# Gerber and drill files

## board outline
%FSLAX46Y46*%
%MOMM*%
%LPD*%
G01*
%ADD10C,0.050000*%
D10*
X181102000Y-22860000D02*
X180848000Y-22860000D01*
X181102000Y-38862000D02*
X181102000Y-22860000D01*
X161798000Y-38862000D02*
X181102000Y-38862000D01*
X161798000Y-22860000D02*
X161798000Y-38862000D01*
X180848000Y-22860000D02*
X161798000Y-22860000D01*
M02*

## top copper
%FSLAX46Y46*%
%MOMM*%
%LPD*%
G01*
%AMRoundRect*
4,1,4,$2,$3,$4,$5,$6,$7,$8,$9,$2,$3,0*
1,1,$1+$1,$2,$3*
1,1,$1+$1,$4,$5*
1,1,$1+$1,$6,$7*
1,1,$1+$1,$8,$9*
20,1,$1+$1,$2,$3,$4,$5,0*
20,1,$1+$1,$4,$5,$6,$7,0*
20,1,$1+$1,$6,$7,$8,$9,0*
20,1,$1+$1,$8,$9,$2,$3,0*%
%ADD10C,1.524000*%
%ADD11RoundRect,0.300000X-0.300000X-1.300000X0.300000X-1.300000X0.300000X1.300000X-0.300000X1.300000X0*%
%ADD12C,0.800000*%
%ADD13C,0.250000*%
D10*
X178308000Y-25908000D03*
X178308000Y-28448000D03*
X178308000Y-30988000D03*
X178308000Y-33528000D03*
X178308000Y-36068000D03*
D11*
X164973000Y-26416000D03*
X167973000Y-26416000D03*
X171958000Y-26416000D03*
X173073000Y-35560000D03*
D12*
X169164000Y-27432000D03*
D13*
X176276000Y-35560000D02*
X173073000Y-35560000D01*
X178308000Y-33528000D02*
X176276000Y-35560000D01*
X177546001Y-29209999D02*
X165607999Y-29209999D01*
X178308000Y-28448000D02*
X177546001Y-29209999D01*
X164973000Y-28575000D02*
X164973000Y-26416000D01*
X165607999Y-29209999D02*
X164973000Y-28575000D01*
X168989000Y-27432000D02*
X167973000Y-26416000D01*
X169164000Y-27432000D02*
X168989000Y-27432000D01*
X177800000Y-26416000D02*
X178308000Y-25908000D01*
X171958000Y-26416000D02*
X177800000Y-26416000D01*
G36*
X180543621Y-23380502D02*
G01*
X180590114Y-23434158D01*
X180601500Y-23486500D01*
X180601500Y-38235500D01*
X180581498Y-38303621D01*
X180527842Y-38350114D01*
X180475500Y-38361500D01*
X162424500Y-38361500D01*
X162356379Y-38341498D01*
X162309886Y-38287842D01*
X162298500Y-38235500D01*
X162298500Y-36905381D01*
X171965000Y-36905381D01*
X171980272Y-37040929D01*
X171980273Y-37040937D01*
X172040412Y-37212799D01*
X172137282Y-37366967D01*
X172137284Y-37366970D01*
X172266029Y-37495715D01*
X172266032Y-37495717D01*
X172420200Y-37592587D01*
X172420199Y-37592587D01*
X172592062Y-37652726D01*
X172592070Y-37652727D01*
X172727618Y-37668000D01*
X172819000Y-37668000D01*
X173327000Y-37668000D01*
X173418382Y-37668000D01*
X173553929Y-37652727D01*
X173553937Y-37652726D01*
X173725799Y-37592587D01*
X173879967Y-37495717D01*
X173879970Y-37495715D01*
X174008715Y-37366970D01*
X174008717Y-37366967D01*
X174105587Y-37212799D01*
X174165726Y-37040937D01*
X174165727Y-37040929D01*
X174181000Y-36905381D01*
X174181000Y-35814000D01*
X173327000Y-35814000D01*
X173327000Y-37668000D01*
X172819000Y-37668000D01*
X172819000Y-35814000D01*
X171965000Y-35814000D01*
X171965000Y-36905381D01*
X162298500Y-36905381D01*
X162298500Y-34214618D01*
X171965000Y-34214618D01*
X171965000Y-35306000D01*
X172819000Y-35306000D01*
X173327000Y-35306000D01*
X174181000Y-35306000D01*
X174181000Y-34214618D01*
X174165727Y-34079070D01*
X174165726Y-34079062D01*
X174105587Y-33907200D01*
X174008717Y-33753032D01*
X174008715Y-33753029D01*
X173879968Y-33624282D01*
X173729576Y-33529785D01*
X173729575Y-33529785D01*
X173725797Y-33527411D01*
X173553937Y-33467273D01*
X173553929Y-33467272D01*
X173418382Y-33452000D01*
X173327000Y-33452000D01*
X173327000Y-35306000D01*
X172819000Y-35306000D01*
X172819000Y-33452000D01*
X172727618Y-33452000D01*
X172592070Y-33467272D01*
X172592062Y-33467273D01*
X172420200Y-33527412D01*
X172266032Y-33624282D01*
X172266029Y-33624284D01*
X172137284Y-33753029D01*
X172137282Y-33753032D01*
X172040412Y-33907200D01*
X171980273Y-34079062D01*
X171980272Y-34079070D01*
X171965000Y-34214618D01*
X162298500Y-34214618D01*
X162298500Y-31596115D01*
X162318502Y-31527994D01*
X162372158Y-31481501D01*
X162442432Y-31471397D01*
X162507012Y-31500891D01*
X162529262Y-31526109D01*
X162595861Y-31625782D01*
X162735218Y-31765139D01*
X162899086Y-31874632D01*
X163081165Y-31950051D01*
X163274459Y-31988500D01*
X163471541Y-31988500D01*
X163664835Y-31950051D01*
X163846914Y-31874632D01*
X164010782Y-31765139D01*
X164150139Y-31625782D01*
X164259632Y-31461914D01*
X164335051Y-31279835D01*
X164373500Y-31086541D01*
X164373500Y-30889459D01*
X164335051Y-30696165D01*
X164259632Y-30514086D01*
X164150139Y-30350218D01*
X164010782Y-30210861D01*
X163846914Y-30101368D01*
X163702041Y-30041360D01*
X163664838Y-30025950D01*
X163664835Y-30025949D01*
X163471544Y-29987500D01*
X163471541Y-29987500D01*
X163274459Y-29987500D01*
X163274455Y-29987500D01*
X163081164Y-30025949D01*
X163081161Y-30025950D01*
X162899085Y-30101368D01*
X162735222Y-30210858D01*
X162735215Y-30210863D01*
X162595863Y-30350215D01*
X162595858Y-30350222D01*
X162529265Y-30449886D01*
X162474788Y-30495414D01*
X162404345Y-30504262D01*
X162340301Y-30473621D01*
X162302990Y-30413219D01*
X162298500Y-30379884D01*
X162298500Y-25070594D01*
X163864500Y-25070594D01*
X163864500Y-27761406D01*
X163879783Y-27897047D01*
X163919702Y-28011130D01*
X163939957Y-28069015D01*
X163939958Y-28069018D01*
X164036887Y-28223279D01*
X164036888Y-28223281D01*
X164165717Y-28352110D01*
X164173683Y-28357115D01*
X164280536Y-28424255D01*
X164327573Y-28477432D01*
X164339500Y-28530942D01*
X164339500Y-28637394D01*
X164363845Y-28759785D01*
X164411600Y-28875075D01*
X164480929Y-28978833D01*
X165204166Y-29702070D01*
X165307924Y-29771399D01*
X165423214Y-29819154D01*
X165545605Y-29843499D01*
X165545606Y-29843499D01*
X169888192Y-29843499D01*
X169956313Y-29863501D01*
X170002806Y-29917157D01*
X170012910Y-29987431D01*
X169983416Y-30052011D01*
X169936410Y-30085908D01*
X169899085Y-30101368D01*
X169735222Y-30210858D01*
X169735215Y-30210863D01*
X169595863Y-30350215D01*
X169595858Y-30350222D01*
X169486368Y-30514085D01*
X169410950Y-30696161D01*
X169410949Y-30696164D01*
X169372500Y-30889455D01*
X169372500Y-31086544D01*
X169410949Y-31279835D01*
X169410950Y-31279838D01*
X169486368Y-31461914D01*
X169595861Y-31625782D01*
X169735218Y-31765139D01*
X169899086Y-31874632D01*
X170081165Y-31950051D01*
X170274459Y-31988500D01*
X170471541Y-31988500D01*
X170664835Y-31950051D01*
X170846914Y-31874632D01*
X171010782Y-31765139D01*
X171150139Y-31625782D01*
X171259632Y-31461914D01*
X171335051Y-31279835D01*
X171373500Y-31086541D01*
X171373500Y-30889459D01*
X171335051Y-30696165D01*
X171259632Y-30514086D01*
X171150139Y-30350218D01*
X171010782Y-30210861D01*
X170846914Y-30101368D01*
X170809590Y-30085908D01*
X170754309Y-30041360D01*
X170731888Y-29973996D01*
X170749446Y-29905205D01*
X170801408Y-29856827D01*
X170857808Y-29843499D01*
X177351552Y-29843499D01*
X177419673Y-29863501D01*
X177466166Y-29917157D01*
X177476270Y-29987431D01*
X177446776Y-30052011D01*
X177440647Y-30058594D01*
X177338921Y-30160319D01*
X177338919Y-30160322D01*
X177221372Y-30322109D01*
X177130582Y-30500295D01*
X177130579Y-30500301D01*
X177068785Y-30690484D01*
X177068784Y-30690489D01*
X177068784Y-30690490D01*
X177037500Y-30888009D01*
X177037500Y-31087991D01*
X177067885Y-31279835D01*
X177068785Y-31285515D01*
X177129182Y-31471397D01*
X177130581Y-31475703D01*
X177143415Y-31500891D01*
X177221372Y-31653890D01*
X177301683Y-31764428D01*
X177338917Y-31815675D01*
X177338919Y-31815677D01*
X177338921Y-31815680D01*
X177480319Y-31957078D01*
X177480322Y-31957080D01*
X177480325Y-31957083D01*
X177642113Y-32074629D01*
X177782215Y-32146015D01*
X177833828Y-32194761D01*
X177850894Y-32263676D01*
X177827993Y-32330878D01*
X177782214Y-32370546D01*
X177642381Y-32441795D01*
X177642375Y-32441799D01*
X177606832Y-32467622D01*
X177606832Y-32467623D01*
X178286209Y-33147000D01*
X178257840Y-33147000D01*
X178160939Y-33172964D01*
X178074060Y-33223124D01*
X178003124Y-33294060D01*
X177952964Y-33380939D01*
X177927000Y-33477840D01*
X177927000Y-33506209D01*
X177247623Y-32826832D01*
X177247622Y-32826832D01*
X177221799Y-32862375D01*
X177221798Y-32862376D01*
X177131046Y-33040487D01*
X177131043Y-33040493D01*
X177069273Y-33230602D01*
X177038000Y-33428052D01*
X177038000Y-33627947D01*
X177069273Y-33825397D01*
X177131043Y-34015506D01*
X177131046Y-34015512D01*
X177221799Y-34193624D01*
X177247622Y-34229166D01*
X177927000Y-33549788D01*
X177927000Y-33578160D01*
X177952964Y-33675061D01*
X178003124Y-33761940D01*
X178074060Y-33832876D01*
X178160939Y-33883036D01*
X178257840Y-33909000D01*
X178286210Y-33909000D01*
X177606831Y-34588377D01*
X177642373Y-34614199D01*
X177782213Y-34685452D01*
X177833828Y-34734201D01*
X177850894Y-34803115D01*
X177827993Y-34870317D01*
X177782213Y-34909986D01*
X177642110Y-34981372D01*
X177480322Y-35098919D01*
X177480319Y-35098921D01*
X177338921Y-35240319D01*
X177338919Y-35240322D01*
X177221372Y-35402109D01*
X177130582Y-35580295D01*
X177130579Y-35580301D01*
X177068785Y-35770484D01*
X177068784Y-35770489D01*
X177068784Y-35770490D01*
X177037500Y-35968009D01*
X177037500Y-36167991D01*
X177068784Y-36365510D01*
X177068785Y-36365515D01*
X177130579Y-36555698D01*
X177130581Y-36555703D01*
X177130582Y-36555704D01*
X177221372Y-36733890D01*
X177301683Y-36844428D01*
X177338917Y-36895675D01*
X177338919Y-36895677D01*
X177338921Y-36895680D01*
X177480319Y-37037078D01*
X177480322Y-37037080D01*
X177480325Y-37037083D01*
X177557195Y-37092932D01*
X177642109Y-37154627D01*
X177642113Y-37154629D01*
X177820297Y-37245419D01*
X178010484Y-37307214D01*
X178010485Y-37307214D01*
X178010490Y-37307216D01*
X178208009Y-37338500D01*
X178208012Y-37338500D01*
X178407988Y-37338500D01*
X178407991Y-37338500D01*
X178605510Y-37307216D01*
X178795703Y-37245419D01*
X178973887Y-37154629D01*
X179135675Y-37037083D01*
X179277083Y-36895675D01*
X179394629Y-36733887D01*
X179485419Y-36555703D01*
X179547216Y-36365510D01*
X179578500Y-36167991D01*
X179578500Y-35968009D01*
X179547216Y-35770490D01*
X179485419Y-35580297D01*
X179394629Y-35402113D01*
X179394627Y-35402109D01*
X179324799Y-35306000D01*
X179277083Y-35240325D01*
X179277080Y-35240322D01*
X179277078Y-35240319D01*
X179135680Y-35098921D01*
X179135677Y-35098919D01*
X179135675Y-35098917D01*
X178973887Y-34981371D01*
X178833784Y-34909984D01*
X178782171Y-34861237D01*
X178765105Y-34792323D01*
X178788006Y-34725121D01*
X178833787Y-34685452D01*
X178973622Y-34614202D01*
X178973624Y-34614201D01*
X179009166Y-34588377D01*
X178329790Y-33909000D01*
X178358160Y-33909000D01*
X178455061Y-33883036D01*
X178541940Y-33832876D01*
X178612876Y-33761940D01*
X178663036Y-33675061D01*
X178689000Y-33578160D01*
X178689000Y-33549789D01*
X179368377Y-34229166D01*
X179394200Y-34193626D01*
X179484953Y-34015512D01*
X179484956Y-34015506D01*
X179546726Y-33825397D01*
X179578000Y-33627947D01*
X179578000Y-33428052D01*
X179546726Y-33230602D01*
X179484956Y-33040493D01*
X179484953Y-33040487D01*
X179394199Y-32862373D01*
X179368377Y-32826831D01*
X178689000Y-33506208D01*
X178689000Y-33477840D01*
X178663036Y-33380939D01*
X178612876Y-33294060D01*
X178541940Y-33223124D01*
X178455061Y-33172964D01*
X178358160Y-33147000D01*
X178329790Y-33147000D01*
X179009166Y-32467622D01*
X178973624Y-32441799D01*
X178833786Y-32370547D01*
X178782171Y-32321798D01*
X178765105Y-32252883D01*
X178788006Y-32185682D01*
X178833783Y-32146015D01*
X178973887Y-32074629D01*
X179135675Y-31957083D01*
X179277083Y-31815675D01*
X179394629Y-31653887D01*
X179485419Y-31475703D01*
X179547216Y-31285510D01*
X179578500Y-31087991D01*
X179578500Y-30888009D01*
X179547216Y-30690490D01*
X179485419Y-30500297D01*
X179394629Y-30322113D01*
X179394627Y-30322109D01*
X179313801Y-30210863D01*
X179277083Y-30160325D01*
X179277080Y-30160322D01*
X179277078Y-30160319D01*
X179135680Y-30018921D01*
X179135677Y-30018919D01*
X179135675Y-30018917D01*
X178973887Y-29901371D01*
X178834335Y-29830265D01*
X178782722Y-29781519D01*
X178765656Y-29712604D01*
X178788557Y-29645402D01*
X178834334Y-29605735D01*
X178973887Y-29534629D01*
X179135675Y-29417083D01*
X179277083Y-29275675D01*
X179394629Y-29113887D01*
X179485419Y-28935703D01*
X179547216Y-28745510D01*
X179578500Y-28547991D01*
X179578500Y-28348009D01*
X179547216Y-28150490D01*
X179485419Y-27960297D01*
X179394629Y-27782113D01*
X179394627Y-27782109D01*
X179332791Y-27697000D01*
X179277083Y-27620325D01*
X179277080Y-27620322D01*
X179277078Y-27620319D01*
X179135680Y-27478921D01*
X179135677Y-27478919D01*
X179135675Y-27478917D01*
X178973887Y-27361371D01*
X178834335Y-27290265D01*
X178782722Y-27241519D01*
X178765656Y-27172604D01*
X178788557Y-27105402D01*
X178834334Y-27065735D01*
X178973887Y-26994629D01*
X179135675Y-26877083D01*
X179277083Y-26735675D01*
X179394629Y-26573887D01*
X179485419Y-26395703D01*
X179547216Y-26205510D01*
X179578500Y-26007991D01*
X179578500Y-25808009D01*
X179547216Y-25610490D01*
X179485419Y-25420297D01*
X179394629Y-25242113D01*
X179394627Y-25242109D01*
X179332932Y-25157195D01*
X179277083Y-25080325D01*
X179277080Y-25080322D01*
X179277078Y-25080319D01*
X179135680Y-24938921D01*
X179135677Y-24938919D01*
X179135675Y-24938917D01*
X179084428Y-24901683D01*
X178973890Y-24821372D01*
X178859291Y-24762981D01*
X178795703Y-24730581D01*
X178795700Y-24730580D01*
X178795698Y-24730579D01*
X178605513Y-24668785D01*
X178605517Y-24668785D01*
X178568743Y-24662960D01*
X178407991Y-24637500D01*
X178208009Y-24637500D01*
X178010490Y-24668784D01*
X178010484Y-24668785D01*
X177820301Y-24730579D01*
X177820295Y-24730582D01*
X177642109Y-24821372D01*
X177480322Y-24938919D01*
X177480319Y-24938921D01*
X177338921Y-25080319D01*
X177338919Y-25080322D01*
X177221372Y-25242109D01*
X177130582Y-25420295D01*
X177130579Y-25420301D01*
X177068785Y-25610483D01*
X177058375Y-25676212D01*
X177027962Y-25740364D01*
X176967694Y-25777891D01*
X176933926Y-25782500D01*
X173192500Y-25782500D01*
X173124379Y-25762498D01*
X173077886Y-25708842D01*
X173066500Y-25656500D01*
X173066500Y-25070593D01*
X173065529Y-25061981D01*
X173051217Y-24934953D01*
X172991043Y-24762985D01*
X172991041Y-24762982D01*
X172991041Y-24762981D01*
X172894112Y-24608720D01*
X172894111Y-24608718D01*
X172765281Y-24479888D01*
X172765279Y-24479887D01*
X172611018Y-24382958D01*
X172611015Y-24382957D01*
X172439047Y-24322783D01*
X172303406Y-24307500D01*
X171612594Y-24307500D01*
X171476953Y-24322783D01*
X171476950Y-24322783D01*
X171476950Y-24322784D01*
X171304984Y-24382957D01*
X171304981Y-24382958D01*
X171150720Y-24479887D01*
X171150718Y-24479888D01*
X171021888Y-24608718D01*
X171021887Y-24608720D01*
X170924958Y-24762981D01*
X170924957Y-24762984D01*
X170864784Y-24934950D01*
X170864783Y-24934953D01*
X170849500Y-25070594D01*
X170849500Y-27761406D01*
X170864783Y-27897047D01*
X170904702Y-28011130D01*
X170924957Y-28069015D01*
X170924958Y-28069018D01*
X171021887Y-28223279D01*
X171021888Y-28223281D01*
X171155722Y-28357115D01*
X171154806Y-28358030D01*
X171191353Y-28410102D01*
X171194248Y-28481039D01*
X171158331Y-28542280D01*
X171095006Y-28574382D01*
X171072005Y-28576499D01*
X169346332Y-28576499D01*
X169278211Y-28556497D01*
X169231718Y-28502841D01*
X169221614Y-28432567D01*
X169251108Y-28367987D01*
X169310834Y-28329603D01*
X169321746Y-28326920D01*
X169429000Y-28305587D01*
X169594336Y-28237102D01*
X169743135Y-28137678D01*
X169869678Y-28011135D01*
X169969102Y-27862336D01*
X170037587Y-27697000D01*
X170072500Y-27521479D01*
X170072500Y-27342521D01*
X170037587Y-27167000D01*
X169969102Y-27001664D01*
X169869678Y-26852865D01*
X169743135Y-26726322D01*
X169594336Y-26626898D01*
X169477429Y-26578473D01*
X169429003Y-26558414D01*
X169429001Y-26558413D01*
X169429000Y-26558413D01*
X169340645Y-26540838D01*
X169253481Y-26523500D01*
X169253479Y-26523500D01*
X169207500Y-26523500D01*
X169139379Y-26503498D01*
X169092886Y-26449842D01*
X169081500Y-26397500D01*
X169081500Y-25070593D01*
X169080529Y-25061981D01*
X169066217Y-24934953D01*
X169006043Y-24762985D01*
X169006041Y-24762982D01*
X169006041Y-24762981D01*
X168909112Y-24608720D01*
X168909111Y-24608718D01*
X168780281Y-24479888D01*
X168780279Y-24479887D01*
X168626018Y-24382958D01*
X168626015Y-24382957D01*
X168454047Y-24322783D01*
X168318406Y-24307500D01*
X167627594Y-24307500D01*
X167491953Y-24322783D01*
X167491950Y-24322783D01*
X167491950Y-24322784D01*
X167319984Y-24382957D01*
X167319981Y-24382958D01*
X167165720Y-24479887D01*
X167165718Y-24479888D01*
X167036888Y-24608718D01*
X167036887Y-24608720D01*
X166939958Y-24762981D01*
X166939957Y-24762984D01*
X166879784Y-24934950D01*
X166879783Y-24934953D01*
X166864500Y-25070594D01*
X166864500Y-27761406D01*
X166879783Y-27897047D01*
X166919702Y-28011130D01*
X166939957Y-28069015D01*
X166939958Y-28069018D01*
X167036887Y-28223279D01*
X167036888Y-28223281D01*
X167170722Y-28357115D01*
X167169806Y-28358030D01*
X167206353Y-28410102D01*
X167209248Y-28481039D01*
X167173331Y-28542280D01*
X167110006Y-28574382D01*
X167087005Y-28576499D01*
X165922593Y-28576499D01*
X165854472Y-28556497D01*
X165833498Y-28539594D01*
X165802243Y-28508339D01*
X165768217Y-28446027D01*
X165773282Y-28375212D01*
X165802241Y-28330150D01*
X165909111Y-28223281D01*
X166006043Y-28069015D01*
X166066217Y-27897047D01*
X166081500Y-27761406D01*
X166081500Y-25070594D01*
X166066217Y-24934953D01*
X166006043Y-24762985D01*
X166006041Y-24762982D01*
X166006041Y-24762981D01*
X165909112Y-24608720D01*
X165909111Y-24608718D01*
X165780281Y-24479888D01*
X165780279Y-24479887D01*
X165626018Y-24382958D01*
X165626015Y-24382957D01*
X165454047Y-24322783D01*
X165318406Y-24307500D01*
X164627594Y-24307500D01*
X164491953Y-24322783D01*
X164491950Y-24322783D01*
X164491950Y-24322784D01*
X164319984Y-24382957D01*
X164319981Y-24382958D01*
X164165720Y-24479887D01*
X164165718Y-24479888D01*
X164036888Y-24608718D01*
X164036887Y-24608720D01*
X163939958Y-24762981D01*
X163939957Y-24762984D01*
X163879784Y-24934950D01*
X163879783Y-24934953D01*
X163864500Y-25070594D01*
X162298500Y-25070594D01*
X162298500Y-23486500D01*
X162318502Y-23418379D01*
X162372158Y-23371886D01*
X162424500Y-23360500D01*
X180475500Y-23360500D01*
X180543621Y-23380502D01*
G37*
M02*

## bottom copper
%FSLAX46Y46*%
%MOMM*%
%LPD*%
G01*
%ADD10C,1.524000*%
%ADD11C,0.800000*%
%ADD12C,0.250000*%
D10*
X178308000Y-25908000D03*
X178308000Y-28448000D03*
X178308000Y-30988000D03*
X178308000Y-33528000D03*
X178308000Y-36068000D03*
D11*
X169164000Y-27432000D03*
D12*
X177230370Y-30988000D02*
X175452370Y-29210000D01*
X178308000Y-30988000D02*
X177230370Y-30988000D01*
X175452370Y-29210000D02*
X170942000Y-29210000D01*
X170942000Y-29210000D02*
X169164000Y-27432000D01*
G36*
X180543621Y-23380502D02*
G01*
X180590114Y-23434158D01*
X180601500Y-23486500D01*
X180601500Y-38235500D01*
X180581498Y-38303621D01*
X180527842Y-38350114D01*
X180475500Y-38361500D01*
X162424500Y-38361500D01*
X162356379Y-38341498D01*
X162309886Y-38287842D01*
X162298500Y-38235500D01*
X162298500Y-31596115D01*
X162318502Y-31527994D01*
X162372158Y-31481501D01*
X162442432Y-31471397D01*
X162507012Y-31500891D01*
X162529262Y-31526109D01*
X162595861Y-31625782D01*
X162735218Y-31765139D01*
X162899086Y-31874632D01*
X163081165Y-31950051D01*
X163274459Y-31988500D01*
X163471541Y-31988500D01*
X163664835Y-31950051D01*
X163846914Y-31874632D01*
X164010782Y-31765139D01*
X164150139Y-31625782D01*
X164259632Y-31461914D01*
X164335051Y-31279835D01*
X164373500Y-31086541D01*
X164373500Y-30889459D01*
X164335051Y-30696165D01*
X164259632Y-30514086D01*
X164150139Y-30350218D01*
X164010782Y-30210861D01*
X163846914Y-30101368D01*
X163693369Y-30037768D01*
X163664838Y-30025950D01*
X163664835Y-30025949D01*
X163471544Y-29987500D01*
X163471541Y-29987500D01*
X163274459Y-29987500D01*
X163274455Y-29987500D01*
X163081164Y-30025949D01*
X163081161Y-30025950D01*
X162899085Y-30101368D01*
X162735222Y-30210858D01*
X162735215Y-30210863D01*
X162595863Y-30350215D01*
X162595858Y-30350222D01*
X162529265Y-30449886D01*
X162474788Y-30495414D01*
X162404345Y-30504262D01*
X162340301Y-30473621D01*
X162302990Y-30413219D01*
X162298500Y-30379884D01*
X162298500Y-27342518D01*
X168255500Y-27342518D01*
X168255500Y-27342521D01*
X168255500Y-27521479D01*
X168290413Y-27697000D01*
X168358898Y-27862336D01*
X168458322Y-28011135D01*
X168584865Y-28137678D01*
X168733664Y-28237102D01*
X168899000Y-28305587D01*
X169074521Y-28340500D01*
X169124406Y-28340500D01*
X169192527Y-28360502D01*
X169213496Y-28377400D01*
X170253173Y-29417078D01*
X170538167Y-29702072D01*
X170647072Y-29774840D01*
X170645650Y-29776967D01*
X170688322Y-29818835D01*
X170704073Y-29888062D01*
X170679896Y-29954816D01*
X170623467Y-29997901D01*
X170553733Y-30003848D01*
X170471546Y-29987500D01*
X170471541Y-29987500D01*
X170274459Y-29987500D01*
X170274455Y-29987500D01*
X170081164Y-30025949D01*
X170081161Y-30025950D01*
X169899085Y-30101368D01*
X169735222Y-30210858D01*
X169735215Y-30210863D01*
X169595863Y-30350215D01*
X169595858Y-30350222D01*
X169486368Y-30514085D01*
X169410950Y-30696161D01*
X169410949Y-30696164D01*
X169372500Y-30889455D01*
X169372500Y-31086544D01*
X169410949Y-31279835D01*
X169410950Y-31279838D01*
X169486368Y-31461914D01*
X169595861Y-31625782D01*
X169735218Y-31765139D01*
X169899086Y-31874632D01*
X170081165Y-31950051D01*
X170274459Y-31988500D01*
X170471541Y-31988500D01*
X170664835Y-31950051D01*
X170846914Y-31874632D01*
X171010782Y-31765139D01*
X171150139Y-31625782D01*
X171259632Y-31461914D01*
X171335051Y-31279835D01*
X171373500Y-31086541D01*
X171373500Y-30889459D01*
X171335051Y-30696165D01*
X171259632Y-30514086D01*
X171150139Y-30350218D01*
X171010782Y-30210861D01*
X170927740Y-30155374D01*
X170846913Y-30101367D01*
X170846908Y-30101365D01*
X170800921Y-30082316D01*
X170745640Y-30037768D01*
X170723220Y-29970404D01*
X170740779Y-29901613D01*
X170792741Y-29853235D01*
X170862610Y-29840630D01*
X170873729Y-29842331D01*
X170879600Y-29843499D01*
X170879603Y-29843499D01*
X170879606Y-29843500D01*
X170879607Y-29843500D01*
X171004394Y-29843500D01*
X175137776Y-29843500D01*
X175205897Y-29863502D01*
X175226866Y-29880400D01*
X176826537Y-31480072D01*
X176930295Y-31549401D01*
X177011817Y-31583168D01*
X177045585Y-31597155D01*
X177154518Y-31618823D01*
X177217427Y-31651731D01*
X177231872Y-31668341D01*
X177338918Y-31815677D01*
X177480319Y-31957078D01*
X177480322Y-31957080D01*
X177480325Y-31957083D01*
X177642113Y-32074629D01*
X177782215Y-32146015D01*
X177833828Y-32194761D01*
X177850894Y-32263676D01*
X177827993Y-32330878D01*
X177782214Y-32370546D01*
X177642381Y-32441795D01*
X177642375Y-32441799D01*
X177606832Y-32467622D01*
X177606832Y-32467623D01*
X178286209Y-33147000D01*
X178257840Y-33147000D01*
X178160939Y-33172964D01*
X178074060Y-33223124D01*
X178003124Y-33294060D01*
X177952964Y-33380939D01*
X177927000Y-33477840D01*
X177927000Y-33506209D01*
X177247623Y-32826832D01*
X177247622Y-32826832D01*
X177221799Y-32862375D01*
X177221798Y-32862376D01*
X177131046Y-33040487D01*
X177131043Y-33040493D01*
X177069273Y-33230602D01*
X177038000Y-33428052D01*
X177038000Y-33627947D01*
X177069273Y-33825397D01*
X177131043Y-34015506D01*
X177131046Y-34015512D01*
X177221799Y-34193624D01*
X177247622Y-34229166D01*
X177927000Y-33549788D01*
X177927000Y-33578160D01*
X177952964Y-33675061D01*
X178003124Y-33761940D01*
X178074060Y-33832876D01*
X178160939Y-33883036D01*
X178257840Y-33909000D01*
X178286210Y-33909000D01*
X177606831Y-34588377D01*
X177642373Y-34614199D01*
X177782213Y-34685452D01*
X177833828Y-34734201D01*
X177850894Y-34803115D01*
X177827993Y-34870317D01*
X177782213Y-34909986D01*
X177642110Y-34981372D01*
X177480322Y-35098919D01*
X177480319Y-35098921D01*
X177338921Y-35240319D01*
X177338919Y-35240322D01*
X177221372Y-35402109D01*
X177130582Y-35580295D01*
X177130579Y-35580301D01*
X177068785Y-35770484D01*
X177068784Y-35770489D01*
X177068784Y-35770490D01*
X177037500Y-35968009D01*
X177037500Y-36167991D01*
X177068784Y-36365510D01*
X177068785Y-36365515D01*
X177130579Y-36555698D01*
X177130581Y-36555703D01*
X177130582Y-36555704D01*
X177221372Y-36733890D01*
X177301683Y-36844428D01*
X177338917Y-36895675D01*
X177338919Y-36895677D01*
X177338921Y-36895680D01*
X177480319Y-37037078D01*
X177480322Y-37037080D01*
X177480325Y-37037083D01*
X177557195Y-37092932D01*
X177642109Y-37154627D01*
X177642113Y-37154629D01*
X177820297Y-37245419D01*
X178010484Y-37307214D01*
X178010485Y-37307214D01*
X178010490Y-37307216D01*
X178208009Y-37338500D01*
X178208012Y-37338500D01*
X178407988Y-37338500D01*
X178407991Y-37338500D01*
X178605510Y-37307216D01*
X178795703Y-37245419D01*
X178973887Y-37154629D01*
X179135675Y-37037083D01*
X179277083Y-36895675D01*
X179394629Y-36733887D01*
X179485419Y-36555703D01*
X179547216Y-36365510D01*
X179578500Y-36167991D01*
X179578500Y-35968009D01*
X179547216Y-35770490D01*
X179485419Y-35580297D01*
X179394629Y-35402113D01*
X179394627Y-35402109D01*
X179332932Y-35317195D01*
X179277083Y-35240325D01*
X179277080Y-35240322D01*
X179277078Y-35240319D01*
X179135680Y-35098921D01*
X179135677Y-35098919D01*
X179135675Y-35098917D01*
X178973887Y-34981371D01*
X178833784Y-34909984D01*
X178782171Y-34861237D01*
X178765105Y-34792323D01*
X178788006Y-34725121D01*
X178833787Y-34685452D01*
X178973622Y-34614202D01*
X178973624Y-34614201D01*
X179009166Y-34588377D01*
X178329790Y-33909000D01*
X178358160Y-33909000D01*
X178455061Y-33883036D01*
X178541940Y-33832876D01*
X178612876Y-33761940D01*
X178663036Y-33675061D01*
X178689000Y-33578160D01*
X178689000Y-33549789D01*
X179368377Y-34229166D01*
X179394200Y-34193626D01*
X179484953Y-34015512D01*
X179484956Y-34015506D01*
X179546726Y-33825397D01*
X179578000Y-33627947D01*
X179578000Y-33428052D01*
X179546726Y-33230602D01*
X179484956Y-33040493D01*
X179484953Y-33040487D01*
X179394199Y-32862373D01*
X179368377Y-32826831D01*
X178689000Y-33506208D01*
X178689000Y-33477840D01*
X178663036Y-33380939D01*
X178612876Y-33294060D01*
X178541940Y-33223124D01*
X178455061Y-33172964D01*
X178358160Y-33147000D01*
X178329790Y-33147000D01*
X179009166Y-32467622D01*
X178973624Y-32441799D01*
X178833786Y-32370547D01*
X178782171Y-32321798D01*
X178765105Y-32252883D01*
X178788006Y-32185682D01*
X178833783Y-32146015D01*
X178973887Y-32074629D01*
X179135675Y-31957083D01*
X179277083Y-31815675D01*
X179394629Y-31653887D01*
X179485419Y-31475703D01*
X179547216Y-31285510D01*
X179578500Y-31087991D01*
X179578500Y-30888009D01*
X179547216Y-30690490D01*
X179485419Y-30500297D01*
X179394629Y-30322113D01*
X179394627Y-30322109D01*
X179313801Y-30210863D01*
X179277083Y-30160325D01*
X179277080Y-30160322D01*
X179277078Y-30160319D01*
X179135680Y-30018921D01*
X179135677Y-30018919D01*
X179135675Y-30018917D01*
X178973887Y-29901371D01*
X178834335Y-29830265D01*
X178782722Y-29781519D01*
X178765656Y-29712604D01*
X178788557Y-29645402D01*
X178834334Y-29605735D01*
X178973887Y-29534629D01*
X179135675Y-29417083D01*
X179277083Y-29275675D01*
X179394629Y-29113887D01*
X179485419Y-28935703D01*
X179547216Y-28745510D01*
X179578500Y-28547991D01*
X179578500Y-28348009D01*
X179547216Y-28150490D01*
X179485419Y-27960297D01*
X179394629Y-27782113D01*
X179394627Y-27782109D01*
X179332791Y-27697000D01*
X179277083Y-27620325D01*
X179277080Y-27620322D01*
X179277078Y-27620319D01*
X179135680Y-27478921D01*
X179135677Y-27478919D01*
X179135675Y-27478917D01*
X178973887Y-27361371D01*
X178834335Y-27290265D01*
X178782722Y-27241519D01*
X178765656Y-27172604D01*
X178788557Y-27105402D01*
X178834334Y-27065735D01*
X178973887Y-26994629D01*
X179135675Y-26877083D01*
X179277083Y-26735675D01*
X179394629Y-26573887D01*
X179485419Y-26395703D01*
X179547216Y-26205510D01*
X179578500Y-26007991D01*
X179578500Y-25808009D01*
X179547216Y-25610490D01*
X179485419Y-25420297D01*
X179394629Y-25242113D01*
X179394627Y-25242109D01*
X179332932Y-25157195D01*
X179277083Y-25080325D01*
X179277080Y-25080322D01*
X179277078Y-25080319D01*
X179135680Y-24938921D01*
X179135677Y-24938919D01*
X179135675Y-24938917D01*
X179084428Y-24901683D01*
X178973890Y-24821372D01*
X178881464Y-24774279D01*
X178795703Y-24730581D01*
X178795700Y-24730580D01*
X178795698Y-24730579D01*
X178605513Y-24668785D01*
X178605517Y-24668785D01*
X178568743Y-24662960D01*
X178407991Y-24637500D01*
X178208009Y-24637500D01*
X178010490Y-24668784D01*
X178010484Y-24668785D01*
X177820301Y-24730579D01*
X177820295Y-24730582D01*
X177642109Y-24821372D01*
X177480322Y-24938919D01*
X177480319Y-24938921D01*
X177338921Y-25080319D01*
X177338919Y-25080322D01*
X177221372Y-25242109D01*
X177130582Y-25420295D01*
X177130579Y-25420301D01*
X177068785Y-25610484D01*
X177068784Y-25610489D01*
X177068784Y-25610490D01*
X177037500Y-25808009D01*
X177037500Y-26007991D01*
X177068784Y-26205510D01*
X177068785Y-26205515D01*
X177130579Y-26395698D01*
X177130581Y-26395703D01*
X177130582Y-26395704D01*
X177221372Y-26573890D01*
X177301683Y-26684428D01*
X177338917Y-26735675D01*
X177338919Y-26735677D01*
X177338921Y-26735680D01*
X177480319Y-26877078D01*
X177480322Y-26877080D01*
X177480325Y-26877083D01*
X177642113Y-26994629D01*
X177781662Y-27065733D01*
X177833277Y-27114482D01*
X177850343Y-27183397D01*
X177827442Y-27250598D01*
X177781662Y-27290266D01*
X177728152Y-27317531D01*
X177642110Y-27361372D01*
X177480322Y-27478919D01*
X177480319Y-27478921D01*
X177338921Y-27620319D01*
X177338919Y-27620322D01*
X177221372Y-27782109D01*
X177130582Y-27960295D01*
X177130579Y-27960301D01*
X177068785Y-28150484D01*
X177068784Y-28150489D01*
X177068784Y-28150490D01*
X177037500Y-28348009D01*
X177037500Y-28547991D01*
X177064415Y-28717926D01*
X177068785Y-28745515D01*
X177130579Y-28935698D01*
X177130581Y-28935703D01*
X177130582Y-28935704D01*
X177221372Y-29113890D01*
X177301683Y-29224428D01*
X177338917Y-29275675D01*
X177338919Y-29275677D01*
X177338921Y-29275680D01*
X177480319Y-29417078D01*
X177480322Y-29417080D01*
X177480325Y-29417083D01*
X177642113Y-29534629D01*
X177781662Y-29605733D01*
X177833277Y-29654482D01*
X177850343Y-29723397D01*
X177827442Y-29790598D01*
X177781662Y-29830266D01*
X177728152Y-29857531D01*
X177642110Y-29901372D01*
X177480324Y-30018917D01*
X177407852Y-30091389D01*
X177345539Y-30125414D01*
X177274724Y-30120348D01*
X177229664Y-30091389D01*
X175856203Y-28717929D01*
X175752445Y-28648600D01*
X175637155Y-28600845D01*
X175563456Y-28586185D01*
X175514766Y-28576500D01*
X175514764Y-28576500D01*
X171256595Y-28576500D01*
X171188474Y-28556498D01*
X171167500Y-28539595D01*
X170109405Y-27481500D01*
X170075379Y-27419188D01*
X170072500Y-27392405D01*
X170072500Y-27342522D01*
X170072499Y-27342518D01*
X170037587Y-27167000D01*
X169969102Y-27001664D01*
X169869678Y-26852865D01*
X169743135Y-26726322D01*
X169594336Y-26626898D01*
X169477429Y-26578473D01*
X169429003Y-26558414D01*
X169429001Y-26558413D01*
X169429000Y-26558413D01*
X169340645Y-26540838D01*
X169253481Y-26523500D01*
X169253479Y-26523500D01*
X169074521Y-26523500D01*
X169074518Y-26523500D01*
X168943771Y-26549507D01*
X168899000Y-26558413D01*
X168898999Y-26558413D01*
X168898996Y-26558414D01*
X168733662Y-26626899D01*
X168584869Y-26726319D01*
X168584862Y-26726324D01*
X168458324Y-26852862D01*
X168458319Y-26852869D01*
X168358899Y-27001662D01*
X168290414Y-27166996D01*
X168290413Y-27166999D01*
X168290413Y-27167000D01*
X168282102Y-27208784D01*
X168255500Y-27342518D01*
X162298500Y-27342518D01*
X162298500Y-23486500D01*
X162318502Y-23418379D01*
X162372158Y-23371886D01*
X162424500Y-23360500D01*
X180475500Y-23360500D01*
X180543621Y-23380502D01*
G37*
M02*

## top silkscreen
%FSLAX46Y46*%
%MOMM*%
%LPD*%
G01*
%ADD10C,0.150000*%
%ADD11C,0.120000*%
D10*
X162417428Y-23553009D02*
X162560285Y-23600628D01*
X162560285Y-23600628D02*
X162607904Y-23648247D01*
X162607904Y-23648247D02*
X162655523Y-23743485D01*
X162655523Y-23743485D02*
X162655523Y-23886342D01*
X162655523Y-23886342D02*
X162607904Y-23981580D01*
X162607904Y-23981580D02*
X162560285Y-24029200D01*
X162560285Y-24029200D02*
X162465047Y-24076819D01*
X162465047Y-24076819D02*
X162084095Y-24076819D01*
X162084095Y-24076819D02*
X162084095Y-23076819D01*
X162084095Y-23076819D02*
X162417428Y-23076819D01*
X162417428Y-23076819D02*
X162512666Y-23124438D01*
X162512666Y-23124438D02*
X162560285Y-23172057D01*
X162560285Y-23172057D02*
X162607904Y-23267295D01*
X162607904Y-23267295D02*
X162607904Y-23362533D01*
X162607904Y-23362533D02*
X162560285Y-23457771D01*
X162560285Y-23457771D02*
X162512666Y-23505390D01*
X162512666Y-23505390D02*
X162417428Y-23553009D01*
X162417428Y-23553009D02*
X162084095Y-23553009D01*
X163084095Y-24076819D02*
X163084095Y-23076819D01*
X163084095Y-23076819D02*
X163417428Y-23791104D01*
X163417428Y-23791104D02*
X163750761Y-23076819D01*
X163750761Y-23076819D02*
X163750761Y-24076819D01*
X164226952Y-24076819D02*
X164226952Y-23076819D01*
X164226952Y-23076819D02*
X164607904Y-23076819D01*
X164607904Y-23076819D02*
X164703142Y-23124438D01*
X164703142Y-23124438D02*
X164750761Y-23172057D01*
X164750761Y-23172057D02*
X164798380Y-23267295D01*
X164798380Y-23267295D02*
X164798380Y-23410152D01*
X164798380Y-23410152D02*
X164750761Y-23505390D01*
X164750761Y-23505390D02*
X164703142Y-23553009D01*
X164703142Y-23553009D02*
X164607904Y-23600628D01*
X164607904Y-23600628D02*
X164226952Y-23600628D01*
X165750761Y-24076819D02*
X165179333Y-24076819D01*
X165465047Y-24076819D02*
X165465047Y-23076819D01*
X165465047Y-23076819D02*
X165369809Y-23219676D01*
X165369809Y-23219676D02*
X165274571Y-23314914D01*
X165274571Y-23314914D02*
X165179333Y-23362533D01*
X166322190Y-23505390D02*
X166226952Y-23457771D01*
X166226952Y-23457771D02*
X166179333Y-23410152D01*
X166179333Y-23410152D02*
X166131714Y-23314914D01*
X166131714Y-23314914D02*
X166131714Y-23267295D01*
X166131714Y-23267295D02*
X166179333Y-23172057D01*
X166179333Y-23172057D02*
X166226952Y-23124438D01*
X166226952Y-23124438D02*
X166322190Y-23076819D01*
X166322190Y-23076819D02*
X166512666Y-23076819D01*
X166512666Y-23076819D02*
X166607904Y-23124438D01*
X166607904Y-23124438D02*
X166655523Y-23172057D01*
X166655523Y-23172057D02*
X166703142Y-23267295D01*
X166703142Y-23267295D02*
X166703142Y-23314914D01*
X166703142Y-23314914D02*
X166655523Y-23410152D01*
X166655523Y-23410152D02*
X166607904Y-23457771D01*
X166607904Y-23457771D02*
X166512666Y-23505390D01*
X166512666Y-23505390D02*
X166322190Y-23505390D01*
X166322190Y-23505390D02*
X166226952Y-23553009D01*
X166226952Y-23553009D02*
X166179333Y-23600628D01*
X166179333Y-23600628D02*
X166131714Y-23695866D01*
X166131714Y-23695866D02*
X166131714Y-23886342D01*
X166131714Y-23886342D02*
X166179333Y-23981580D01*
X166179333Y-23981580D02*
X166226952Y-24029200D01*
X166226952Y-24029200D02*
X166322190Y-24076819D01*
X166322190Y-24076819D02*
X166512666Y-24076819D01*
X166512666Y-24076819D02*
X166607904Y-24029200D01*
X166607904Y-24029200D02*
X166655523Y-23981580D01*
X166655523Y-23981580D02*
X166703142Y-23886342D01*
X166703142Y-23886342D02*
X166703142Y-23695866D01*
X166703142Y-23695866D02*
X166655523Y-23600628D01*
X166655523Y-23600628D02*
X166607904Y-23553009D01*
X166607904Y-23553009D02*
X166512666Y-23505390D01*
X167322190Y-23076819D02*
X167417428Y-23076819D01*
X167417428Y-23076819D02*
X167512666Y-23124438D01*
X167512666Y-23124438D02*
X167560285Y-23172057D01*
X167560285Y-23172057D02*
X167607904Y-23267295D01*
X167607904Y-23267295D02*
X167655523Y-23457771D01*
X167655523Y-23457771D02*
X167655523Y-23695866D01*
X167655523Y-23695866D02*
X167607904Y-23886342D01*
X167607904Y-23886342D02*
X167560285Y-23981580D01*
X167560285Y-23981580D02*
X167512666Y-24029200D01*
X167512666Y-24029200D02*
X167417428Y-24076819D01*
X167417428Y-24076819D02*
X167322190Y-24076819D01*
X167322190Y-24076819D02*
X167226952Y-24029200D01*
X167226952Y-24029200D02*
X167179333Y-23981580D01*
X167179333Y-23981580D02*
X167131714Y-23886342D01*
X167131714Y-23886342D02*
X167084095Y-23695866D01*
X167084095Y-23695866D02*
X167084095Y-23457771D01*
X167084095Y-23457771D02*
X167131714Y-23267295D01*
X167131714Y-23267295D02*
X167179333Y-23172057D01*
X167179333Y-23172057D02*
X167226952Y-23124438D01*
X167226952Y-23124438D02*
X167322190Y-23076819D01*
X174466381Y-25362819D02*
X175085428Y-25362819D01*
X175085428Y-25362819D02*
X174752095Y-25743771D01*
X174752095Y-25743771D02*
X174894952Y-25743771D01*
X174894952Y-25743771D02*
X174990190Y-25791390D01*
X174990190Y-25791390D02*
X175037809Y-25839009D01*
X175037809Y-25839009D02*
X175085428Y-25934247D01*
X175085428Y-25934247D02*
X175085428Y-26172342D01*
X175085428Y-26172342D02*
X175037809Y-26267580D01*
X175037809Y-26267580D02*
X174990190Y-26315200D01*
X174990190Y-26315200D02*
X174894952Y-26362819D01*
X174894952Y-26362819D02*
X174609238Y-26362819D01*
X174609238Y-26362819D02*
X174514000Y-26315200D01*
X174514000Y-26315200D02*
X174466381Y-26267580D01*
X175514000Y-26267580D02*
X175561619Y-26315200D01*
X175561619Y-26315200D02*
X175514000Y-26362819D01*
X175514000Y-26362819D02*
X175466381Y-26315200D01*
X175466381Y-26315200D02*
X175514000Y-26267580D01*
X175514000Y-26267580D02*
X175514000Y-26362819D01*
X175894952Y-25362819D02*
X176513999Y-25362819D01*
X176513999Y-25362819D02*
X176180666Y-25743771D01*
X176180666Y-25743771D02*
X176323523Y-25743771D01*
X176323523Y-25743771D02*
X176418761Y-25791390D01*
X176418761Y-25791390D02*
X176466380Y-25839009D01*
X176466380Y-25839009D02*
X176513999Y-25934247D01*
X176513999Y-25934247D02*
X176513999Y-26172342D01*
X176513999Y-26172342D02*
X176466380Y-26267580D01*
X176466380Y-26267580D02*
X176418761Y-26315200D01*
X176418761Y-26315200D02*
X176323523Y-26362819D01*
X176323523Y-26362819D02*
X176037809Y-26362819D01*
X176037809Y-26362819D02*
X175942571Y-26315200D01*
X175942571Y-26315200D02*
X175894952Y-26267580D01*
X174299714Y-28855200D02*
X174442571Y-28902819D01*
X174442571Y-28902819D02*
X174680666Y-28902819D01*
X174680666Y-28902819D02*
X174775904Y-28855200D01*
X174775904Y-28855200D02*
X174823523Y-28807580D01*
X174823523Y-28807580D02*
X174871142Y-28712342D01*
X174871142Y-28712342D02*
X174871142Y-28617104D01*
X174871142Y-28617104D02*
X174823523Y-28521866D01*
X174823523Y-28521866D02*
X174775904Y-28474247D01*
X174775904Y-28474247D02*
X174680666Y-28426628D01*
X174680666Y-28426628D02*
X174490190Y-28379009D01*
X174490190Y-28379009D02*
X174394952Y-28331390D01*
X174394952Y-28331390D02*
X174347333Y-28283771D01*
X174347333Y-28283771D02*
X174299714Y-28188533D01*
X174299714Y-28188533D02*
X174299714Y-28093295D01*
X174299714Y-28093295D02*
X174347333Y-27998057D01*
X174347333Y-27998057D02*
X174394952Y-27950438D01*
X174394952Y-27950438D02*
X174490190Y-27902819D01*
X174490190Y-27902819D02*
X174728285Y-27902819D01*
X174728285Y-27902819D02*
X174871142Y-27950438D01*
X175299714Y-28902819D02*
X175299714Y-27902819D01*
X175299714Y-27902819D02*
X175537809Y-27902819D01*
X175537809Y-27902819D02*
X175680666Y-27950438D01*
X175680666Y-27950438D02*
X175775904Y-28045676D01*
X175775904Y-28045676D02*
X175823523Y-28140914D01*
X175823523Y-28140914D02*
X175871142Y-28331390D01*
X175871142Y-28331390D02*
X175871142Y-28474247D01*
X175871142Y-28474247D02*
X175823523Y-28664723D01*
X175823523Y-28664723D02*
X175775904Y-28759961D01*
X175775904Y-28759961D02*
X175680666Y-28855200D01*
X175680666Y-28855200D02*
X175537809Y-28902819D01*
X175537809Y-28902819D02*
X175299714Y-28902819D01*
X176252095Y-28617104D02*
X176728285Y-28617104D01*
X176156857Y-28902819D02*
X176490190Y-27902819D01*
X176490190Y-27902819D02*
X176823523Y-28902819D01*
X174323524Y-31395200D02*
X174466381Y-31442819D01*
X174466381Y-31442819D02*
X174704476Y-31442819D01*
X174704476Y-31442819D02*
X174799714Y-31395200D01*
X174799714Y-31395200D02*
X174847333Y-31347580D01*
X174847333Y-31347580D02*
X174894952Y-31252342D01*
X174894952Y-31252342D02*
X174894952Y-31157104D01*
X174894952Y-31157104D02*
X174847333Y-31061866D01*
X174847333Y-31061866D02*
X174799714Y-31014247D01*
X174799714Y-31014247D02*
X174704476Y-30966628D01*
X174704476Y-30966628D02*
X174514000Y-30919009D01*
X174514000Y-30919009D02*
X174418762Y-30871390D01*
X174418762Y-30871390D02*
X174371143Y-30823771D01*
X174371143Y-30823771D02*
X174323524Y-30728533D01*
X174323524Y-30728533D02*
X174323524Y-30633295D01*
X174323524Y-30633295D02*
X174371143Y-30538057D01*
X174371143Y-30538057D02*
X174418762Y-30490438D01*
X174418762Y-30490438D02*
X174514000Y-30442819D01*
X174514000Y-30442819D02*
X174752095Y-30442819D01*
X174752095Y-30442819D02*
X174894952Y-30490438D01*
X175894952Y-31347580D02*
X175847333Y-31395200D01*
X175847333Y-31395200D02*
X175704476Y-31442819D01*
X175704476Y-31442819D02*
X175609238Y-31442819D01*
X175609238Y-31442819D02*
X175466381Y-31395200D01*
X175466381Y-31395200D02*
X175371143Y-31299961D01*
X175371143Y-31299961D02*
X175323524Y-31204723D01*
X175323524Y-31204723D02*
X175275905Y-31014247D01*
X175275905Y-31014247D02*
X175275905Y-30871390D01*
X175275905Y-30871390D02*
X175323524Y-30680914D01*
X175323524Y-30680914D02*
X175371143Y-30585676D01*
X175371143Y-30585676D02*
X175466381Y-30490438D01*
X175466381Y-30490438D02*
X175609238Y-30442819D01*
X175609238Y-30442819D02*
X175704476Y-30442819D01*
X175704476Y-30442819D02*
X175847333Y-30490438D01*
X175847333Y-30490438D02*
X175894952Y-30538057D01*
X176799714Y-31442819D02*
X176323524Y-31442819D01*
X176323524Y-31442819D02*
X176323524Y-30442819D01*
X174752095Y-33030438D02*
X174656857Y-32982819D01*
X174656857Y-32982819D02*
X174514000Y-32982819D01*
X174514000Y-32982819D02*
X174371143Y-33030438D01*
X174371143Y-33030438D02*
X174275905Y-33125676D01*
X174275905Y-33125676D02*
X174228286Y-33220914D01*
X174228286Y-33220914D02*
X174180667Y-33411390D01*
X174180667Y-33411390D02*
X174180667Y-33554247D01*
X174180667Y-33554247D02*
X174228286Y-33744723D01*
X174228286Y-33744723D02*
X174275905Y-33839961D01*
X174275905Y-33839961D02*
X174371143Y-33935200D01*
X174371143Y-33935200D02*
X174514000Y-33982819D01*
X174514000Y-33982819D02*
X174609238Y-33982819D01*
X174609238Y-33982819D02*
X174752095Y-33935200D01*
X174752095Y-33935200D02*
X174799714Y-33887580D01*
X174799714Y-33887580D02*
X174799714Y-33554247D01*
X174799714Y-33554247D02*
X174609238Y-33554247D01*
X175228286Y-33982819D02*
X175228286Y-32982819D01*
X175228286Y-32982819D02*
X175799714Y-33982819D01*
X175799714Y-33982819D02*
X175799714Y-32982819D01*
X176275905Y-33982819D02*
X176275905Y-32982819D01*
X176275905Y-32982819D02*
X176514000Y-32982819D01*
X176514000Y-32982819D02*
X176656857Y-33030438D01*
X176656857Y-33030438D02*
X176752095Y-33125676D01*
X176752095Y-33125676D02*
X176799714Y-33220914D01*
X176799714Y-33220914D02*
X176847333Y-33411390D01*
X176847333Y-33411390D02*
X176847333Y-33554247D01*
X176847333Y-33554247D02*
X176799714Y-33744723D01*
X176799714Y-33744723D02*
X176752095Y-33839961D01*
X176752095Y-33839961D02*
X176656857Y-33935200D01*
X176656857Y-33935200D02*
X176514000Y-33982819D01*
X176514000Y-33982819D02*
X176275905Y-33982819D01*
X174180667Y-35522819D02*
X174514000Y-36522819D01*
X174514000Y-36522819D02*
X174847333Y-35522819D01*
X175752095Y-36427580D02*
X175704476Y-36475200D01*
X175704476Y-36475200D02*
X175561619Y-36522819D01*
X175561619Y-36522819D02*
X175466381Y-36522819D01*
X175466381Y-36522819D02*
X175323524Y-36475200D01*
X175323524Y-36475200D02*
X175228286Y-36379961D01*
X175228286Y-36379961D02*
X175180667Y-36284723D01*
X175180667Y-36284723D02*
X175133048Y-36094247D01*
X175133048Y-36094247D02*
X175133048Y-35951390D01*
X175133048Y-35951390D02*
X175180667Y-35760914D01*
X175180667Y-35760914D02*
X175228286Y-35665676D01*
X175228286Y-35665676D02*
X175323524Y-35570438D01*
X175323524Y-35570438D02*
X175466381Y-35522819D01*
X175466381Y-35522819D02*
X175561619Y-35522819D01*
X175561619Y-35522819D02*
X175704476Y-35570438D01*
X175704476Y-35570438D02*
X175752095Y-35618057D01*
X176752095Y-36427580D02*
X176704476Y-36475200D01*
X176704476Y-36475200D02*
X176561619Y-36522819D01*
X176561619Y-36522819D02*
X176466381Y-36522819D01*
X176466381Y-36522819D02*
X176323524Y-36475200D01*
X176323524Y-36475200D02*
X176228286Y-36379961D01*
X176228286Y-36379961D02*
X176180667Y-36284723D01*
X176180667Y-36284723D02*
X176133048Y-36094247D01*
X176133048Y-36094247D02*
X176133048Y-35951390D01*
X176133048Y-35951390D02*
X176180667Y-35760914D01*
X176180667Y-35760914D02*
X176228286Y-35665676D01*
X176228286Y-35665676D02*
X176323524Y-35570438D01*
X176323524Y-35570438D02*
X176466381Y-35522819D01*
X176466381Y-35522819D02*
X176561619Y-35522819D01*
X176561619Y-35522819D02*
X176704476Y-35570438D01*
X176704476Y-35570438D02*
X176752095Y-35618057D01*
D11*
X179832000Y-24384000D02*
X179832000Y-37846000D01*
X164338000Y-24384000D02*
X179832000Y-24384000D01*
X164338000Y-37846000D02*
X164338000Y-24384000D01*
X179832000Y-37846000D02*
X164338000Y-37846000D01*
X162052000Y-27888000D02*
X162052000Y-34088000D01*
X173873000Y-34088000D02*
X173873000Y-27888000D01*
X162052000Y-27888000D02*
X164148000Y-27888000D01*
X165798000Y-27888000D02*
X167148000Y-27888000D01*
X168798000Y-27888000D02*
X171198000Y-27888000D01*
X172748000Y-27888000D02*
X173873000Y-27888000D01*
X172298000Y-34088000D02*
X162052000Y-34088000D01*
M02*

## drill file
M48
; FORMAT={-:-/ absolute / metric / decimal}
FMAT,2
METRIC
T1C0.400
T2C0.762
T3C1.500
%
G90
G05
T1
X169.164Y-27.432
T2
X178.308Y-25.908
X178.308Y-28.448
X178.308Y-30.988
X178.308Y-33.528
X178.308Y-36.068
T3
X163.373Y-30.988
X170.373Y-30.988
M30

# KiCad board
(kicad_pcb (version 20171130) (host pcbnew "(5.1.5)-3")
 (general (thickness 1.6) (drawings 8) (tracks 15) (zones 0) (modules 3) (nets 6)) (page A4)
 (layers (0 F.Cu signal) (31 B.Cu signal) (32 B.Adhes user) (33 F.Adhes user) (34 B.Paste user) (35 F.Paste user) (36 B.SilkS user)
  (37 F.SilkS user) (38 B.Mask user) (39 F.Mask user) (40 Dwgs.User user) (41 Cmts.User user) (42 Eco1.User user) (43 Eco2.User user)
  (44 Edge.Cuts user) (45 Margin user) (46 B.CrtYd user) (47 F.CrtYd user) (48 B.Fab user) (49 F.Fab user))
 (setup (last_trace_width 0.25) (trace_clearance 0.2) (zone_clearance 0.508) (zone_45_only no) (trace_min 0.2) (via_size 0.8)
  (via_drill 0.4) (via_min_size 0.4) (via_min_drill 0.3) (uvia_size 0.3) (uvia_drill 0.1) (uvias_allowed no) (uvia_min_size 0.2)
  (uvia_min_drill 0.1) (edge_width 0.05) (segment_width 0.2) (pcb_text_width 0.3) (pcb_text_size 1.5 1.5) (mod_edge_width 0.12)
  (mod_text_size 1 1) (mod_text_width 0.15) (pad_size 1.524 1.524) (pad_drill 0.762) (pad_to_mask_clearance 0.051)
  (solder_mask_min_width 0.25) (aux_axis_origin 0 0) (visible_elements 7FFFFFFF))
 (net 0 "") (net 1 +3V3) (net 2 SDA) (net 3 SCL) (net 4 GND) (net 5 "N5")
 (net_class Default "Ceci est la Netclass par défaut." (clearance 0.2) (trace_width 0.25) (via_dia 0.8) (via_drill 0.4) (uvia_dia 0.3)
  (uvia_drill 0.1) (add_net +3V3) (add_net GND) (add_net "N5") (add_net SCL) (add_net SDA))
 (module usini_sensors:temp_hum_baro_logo (layer B.Cu) (at 172.466 27.178 180)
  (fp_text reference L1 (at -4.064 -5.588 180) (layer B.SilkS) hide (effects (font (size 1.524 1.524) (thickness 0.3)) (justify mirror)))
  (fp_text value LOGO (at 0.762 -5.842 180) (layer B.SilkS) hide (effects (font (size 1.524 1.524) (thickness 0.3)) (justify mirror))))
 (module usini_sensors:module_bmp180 (layer F.Cu) (at 178.308 25.908 180)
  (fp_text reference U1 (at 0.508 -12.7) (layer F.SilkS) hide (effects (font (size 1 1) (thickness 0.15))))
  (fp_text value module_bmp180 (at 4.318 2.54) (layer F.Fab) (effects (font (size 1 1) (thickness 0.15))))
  (fp_line (start -1.524 1.524) (end -1.524 -11.938) (layer F.SilkS) (width 0.12))
  (fp_line (start 13.97 1.524) (end -1.524 1.524) (layer F.SilkS) (width 0.12))
  (fp_line (start 13.97 -11.938) (end 13.97 1.524) (layer F.SilkS) (width 0.12))
  (fp_line (start -1.524 -11.938) (end 13.97 -11.938) (layer F.SilkS) (width 0.12))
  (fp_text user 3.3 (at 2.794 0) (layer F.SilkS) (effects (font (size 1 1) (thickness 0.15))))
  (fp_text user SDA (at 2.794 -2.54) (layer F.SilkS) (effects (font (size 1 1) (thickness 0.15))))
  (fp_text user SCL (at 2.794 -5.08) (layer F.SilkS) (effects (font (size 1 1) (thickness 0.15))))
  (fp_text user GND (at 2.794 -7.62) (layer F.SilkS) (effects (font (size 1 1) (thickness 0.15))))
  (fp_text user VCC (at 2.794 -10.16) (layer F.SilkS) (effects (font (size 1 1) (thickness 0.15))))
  (pad 5 thru_hole circle (at 0 0 180) (size 1.524 1.524) (drill 0.762) (layers *.Cu *.Mask) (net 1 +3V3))
  (pad 4 thru_hole circle (at 0 -2.54 180) (size 1.524 1.524) (drill 0.762) (layers *.Cu *.Mask) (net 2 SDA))
  (pad 3 thru_hole circle (at 0 -5.08 180) (size 1.524 1.524) (drill 0.762) (layers *.Cu *.Mask) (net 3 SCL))
  (pad 2 thru_hole circle (at 0 -7.62 180) (size 1.524 1.524) (drill 0.762) (layers *.Cu *.Mask) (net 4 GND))
  (pad 1 thru_hole circle (at 0 -10.16 180) (size 1.524 1.524) (drill 0.762) (layers *.Cu *.Mask) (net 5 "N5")))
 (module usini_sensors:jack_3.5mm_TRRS (layer F.Cu) (at 168.148 30.988)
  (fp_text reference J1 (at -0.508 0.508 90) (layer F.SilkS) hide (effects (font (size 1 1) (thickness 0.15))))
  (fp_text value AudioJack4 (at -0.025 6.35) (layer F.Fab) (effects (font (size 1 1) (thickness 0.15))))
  (fp_line (start -6.096 -3.1) (end -6.096 3.1) (layer F.SilkS) (width 0.12))
  (fp_line (start 5.725 3.1) (end 5.725 -3.1) (layer F.SilkS) (width 0.12))
  (fp_line (start -6.096 -3.1) (end -4 -3.1) (layer F.SilkS) (width 0.12))
  (fp_line (start -2.35 -3.1) (end -1 -3.1) (layer F.SilkS) (width 0.12))
  (fp_line (start 0.65 -3.1) (end 3.05 -3.1) (layer F.SilkS) (width 0.12))
  (fp_line (start 4.6 -3.1) (end 5.725 -3.1) (layer F.SilkS) (width 0.12))
  (fp_line (start 4.15 3.1) (end -6.096 3.1) (layer F.SilkS) (width 0.12))
  (pad "" np_thru_hole circle (at 2.225 0) (size 1.5 1.5) (drill 1.5) (layers *.Cu *.Mask))
  (pad "" np_thru_hole circle (at -4.775 0) (size 1.5 1.5) (drill 1.5) (layers *.Cu *.Mask))
  (pad R2 smd roundrect (at -3.175 -4.572) (size 1.2 3.2) (layers F.Cu F.Paste F.Mask) (roundrect_rratio 0.25) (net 2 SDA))
  (pad R1 smd roundrect (at -0.175 -4.572) (size 1.2 3.2) (layers F.Cu F.Paste F.Mask) (roundrect_rratio 0.25) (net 3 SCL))
  (pad T smd roundrect (at 3.81 -4.572) (size 1.2 3.2) (layers F.Cu F.Paste F.Mask) (roundrect_rratio 0.25) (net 1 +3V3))
  (pad S smd roundrect (at 4.925 4.572) (size 1.2 3.2) (layers F.Cu F.Paste F.Mask) (roundrect_rratio 0.25) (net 4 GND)))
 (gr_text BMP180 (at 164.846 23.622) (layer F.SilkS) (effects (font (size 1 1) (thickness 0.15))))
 (gr_line (start 181.102 22.86) (end 180.848 22.86) (layer Edge.Cuts) (width 0.05))
 (gr_line (start 181.102 38.862) (end 181.102 22.86) (layer Edge.Cuts) (width 0.05))
 (gr_line (start 161.798 38.862) (end 181.102 38.862) (layer Edge.Cuts) (width 0.05))
 (gr_line (start 161.798 22.86) (end 161.798 38.862) (layer Edge.Cuts) (width 0.05))
 (gr_line (start 180.848 22.86) (end 161.798 22.86) (layer Edge.Cuts) (width 0.05))
 (segment (start 176.276 35.56) (end 173.073 35.56) (width 0.25) (layer F.Cu) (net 4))
 (segment (start 178.308 33.528) (end 176.276 35.56) (width 0.25) (layer F.Cu) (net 4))
 (segment (start 177.546001 29.209999) (end 165.607999 29.209999) (width 0.25) (layer F.Cu) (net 2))
 (segment (start 178.308 28.448) (end 177.546001 29.209999) (width 0.25) (layer F.Cu) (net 2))
 (segment (start 164.973 28.575) (end 164.973 26.416) (width 0.25) (layer F.Cu) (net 2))
 (segment (start 165.607999 29.209999) (end 164.973 28.575) (width 0.25) (layer F.Cu) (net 2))
 (segment (start 177.23037 30.988) (end 175.45237 29.21) (width 0.25) (layer B.Cu) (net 3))
 (segment (start 178.308 30.988) (end 177.23037 30.988) (width 0.25) (layer B.Cu) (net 3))
 (via (at 169.164 27.432) (size 0.8) (drill 0.4) (layers F.Cu B.Cu) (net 3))
 (segment (start 175.45237 29.21) (end 170.942 29.21) (width 0.25) (layer B.Cu) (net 3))
 (segment (start 170.942 29.21) (end 169.164 27.432) (width 0.25) (layer B.Cu) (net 3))
 (segment (start 168.989 27.432) (end 167.973 26.416) (width 0.25) (layer F.Cu) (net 3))
 (segment (start 169.164 27.432) (end 168.989 27.432) (width 0.25) (layer F.Cu) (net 3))
 (segment (start 177.8 26.416) (end 178.308 25.908) (width 0.25) (layer F.Cu) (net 1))
 (segment (start 171.958 26.416) (end 177.8 26.416) (width 0.25) (layer F.Cu) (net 1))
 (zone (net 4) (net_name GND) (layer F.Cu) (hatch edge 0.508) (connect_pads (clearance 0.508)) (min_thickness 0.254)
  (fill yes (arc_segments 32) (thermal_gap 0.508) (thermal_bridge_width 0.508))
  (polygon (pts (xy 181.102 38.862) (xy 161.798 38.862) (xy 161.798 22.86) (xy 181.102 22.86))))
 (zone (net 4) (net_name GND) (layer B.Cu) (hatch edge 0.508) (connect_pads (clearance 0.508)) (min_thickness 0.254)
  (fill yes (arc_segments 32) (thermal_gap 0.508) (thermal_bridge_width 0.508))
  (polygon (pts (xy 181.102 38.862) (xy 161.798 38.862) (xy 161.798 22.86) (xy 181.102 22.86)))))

